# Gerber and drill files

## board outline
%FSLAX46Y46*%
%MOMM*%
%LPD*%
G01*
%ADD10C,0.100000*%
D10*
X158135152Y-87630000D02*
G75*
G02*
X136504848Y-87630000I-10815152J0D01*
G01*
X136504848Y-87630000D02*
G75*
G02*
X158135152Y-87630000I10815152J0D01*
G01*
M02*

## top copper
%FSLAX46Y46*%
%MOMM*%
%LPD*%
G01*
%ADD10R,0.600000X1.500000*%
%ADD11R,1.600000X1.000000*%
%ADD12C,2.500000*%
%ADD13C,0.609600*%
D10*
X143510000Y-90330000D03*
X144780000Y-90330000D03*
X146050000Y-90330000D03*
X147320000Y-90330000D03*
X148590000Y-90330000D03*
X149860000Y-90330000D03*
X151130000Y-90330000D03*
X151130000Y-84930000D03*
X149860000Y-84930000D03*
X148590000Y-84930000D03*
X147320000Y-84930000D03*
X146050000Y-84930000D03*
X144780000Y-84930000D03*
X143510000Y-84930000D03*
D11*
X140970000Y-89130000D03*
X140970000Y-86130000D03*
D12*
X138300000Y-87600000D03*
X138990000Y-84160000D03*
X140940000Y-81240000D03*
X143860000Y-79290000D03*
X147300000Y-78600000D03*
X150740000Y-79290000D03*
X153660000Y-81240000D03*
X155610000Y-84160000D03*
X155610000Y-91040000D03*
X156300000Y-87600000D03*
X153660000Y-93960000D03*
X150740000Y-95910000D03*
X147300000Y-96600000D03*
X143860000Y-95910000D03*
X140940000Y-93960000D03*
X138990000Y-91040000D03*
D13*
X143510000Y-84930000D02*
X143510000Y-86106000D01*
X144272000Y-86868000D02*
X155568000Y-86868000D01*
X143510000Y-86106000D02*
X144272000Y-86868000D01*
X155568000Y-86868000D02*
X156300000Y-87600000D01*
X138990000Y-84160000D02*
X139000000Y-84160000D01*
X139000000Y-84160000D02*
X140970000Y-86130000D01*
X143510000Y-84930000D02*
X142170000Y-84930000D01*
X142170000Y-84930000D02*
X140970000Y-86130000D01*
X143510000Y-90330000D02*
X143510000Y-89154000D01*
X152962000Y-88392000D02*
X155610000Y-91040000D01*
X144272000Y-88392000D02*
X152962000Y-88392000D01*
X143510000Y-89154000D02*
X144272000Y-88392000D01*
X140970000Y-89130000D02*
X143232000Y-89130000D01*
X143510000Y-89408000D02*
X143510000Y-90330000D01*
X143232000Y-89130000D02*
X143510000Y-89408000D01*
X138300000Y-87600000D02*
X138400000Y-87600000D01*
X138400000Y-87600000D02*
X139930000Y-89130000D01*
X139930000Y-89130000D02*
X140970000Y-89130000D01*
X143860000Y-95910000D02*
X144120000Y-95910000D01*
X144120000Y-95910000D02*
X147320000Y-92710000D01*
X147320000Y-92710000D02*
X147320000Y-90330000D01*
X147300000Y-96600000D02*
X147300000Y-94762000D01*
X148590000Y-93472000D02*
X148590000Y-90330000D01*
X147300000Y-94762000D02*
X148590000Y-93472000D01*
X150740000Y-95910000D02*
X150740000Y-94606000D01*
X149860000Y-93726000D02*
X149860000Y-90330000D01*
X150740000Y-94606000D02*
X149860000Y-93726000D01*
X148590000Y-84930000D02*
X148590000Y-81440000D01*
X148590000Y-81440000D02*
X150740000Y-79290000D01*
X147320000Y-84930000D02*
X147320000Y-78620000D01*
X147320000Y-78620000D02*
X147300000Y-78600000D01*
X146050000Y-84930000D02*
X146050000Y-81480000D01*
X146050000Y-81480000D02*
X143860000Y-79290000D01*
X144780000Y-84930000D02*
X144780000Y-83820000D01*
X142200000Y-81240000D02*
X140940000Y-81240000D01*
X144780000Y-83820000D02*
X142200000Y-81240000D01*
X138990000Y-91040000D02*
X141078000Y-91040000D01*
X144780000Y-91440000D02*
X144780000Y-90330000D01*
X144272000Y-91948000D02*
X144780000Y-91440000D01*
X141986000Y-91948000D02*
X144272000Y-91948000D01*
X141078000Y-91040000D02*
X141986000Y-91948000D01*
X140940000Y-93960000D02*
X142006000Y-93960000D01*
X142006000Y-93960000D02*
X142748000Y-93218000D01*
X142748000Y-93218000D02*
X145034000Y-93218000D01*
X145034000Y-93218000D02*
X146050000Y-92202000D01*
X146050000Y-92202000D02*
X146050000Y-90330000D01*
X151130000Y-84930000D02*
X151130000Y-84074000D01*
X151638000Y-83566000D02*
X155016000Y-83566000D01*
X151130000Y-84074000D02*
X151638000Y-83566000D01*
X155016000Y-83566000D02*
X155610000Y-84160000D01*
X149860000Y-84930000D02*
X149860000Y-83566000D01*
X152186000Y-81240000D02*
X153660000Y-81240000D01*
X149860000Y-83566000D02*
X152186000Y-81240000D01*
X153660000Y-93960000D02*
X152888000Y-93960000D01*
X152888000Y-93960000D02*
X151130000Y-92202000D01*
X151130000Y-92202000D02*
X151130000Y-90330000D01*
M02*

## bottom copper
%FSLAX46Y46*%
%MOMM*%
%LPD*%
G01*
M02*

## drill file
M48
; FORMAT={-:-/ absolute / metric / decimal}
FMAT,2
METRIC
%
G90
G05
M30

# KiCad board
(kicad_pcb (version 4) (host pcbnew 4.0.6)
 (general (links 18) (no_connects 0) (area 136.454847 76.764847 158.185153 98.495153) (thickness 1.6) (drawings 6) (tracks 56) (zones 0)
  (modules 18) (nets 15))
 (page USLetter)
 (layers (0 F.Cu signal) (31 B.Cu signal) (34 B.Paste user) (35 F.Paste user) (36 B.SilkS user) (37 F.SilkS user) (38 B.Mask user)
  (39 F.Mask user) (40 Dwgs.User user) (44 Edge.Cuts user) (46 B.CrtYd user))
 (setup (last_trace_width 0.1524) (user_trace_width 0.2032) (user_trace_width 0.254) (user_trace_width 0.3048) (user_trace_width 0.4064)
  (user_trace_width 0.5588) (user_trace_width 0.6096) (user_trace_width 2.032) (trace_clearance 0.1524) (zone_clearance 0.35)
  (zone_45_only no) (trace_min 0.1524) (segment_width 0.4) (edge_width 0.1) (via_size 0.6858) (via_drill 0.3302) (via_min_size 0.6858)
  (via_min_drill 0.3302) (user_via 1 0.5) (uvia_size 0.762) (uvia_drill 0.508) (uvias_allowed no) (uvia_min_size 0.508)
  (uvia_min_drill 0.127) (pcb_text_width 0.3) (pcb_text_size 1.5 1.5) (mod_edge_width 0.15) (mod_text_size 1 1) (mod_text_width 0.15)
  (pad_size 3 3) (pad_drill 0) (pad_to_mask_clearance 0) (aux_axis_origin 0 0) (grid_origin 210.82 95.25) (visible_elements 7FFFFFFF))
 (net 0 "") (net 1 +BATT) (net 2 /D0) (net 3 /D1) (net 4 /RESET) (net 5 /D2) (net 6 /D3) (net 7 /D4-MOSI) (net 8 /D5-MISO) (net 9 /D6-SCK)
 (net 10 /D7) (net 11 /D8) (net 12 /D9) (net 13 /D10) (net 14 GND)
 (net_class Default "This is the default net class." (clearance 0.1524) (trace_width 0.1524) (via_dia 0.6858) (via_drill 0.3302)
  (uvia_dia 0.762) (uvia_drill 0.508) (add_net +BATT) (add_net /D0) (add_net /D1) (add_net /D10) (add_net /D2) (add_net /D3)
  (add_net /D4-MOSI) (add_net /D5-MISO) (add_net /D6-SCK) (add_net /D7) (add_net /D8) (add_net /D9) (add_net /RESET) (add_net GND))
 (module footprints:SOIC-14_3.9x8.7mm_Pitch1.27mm (layer F.Cu) (at 147.32 87.63 90)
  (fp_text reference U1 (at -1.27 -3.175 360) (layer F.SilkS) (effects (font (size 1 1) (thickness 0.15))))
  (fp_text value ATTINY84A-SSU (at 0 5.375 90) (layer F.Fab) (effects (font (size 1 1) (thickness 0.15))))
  (pad 1 smd rect (at -2.7 -3.81 90) (size 1.5 0.6) (layers F.Cu F.Paste F.Mask) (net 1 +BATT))
  (pad 2 smd rect (at -2.7 -2.54 90) (size 1.5 0.6) (layers F.Cu F.Paste F.Mask) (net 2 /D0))
  (pad 3 smd rect (at -2.7 -1.27 90) (size 1.5 0.6) (layers F.Cu F.Paste F.Mask) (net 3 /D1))
  (pad 4 smd rect (at -2.7 0 90) (size 1.5 0.6) (layers F.Cu F.Paste F.Mask) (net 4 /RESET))
  (pad 5 smd rect (at -2.7 1.27 90) (size 1.5 0.6) (layers F.Cu F.Paste F.Mask) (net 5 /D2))
  (pad 6 smd rect (at -2.7 2.54 90) (size 1.5 0.6) (layers F.Cu F.Paste F.Mask) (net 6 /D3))
  (pad 7 smd rect (at -2.7 3.81 90) (size 1.5 0.6) (layers F.Cu F.Paste F.Mask) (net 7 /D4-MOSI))
  (pad 8 smd rect (at 2.7 3.81 90) (size 1.5 0.6) (layers F.Cu F.Paste F.Mask) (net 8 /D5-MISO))
  (pad 9 smd rect (at 2.7 2.54 90) (size 1.5 0.6) (layers F.Cu F.Paste F.Mask) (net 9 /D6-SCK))
  (pad 10 smd rect (at 2.7 1.27 90) (size 1.5 0.6) (layers F.Cu F.Paste F.Mask) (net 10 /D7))
  (pad 11 smd rect (at 2.7 0 90) (size 1.5 0.6) (layers F.Cu F.Paste F.Mask) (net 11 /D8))
  (pad 12 smd rect (at 2.7 -1.27 90) (size 1.5 0.6) (layers F.Cu F.Paste F.Mask) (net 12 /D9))
  (pad 13 smd rect (at 2.7 -2.54 90) (size 1.5 0.6) (layers F.Cu F.Paste F.Mask) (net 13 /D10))
  (pad 14 smd rect (at 2.7 -3.81 90) (size 1.5 0.6) (layers F.Cu F.Paste F.Mask) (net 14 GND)))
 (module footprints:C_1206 (layer F.Cu) (at 140.97 87.63 90)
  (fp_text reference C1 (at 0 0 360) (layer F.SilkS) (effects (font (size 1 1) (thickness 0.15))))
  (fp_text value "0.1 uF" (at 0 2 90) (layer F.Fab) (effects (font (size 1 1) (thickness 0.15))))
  (pad 1 smd rect (at -1.5 0 90) (size 1 1.6) (layers F.Cu F.Paste F.Mask) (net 1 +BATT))
  (pad 2 smd rect (at 1.5 0 90) (size 1 1.6) (layers F.Cu F.Paste F.Mask) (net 14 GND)))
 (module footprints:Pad (layer F.Cu) (at 138.3 87.6)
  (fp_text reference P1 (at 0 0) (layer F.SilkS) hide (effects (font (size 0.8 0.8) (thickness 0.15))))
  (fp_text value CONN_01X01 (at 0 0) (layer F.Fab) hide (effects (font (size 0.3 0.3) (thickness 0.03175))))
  (pad 1 smd circle (at 0 0) (size 2.5 2.5) (layers F.Cu F.Paste F.Mask) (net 1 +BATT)))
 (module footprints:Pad (layer F.Cu) (at 138.99 84.16)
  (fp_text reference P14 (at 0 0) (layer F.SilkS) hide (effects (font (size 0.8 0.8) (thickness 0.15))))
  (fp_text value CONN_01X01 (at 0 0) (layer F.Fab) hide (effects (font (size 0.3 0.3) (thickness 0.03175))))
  (pad 1 smd circle (at 0 0) (size 2.5 2.5) (layers F.Cu F.Paste F.Mask) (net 14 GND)))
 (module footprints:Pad (layer F.Cu) (at 140.94 81.24)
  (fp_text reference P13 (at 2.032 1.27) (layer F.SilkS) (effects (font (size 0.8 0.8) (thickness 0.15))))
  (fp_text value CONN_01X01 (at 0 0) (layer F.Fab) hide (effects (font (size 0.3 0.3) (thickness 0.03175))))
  (pad 1 smd circle (at 0 0) (size 2.5 2.5) (layers F.Cu F.Paste F.Mask) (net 13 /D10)))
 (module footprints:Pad (layer F.Cu) (at 143.86 79.29)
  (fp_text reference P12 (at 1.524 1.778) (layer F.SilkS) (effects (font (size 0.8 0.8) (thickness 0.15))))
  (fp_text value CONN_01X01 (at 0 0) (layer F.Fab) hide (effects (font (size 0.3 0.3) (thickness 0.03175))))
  (pad 1 smd circle (at 0 0) (size 2.5 2.5) (layers F.Cu F.Paste F.Mask) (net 12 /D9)))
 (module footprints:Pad (layer F.Cu) (at 147.3 78.6)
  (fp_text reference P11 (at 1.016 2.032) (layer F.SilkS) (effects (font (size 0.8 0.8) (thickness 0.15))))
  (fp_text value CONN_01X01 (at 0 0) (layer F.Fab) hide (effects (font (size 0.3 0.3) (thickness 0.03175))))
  (pad 1 smd circle (at 0 0) (size 2.5 2.5) (layers F.Cu F.Paste F.Mask) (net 11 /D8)))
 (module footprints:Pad (layer F.Cu) (at 150.74 79.29)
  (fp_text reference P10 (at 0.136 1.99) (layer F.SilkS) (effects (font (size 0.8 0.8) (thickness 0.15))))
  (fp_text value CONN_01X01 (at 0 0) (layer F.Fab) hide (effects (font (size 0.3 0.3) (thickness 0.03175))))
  (pad 1 smd circle (at 0 0) (size 2.5 2.5) (layers F.Cu F.Paste F.Mask) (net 10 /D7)))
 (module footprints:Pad (layer F.Cu) (at 153.66 81.24)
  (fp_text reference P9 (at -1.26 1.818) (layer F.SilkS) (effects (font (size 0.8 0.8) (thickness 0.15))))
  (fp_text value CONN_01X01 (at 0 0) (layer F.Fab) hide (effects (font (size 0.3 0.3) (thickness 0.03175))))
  (pad 1 smd circle (at 0 0) (size 2.5 2.5) (layers F.Cu F.Paste F.Mask) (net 9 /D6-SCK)))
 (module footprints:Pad (layer F.Cu) (at 155.61 84.16)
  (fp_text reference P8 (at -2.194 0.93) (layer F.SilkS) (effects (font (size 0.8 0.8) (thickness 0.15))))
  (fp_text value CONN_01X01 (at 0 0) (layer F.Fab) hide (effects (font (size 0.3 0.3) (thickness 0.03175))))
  (pad 1 smd circle (at 0 0) (size 2.5 2.5) (layers F.Cu F.Paste F.Mask) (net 8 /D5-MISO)))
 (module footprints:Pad (layer F.Cu) (at 155.61 91.04)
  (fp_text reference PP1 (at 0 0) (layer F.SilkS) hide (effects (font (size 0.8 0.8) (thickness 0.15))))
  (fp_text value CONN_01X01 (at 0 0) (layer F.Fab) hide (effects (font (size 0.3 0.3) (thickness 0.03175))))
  (pad 1 smd circle (at 0 0) (size 2.5 2.5) (layers F.Cu F.Paste F.Mask) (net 1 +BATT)))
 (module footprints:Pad (layer F.Cu) (at 156.3 87.6)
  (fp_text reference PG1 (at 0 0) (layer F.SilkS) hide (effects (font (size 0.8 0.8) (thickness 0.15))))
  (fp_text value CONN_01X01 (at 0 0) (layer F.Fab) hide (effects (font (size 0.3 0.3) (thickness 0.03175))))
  (pad 1 smd circle (at 0 0) (size 2.5 2.5) (layers F.Cu F.Paste F.Mask) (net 14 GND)))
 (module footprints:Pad (layer F.Cu) (at 153.66 93.96)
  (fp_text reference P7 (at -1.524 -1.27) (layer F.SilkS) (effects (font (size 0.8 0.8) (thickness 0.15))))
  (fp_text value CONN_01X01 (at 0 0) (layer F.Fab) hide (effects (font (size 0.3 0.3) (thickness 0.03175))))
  (pad 1 smd circle (at 0 0) (size 2.5 2.5) (layers F.Cu F.Paste F.Mask) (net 7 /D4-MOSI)))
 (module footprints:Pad (layer F.Cu) (at 150.74 95.91)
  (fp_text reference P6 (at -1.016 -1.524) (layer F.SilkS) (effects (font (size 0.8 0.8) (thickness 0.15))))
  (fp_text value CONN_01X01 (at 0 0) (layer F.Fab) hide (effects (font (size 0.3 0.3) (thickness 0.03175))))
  (pad 1 smd circle (at 0 0) (size 2.5 2.5) (layers F.Cu F.Paste F.Mask) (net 6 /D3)))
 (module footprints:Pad (layer F.Cu) (at 147.3 96.6)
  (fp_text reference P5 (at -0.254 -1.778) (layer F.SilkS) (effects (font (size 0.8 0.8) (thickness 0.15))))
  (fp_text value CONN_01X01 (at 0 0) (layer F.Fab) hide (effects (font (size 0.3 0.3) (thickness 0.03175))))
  (pad 1 smd circle (at 0 0) (size 2.5 2.5) (layers F.Cu F.Paste F.Mask) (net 5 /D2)))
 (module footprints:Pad (layer F.Cu) (at 143.86 95.91)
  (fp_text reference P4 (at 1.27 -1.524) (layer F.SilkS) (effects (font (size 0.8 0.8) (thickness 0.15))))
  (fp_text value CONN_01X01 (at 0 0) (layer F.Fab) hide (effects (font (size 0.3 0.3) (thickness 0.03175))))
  (pad 1 smd circle (at 0 0) (size 2.5 2.5) (layers F.Cu F.Paste F.Mask) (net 4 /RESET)))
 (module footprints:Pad (layer F.Cu) (at 140.94 93.96)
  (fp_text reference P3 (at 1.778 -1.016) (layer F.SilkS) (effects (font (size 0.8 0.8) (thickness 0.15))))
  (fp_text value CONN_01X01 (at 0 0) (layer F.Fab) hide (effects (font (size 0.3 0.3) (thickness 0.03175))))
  (pad 1 smd circle (at 0 0) (size 2.5 2.5) (layers F.Cu F.Paste F.Mask) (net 3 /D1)))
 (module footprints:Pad (layer F.Cu) (at 138.99 91.04)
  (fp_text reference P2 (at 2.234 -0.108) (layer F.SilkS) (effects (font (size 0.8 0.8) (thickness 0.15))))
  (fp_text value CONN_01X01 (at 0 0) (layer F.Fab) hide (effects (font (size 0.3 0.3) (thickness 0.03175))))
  (pad 1 smd circle (at 0 0) (size 2.5 2.5) (layers F.Cu F.Paste F.Mask) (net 2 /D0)))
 (gr_circle (center 147.32 87.63) (end 149.098 98.298) (layer Edge.Cuts) (width 0.1))
 (segment (start 143.51 84.93) (end 143.51 86.106) (width 0.6096) (layer F.Cu) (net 14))
 (segment (start 144.272 86.868) (end 155.568 86.868) (width 0.6096) (layer F.Cu) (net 14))
 (segment (start 143.51 86.106) (end 144.272 86.868) (width 0.6096) (layer F.Cu) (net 14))
 (segment (start 155.568 86.868) (end 156.3 87.6) (width 0.6096) (layer F.Cu) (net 14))
 (segment (start 138.99 84.16) (end 139 84.16) (width 0.6096) (layer F.Cu) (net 14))
 (segment (start 139 84.16) (end 140.97 86.13) (width 0.6096) (layer F.Cu) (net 14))
 (segment (start 143.51 84.93) (end 142.17 84.93) (width 0.6096) (layer F.Cu) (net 14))
 (segment (start 142.17 84.93) (end 140.97 86.13) (width 0.6096) (layer F.Cu) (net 14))
 (segment (start 143.51 90.33) (end 143.51 89.154) (width 0.6096) (layer F.Cu) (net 1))
 (segment (start 152.962 88.392) (end 155.61 91.04) (width 0.6096) (layer F.Cu) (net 1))
 (segment (start 144.272 88.392) (end 152.962 88.392) (width 0.6096) (layer F.Cu) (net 1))
 (segment (start 143.51 89.154) (end 144.272 88.392) (width 0.6096) (layer F.Cu) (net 1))
 (segment (start 140.97 89.13) (end 143.232 89.13) (width 0.6096) (layer F.Cu) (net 1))
 (segment (start 143.51 89.408) (end 143.51 90.33) (width 0.6096) (layer F.Cu) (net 1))
 (segment (start 143.232 89.13) (end 143.51 89.408) (width 0.6096) (layer F.Cu) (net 1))
 (segment (start 138.3 87.6) (end 138.4 87.6) (width 0.6096) (layer F.Cu) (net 1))
 (segment (start 138.4 87.6) (end 139.93 89.13) (width 0.6096) (layer F.Cu) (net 1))
 (segment (start 139.93 89.13) (end 140.97 89.13) (width 0.6096) (layer F.Cu) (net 1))
 (segment (start 143.86 95.91) (end 144.12 95.91) (width 0.6096) (layer F.Cu) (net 4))
 (segment (start 144.12 95.91) (end 147.32 92.71) (width 0.6096) (layer F.Cu) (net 4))
 (segment (start 147.32 92.71) (end 147.32 90.33) (width 0.6096) (layer F.Cu) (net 4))
 (segment (start 147.3 96.6) (end 147.3 94.762) (width 0.6096) (layer F.Cu) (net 5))
 (segment (start 148.59 93.472) (end 148.59 90.33) (width 0.6096) (layer F.Cu) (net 5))
 (segment (start 147.3 94.762) (end 148.59 93.472) (width 0.6096) (layer F.Cu) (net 5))
 (segment (start 150.74 95.91) (end 150.74 94.606) (width 0.6096) (layer F.Cu) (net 6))
 (segment (start 149.86 93.726) (end 149.86 90.33) (width 0.6096) (layer F.Cu) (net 6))
 (segment (start 150.74 94.606) (end 149.86 93.726) (width 0.6096) (layer F.Cu) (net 6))
 (segment (start 148.59 84.93) (end 148.59 81.44) (width 0.6096) (layer F.Cu) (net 10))
 (segment (start 148.59 81.44) (end 150.74 79.29) (width 0.6096) (layer F.Cu) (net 10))
 (segment (start 147.32 84.93) (end 147.32 78.62) (width 0.6096) (layer F.Cu) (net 11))
 (segment (start 147.32 78.62) (end 147.3 78.6) (width 0.6096) (layer F.Cu) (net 11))
 (segment (start 146.05 84.93) (end 146.05 81.48) (width 0.6096) (layer F.Cu) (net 12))
 (segment (start 146.05 81.48) (end 143.86 79.29) (width 0.6096) (layer F.Cu) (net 12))
 (segment (start 144.78 84.93) (end 144.78 83.82) (width 0.6096) (layer F.Cu) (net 13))
 (segment (start 142.2 81.24) (end 140.94 81.24) (width 0.6096) (layer F.Cu) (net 13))
 (segment (start 144.78 83.82) (end 142.2 81.24) (width 0.6096) (layer F.Cu) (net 13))
 (segment (start 138.99 91.04) (end 141.078 91.04) (width 0.6096) (layer F.Cu) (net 2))
 (segment (start 144.78 91.44) (end 144.78 90.33) (width 0.6096) (layer F.Cu) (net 2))
 (segment (start 144.272 91.948) (end 144.78 91.44) (width 0.6096) (layer F.Cu) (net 2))
 (segment (start 141.986 91.948) (end 144.272 91.948) (width 0.6096) (layer F.Cu) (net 2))
 (segment (start 141.078 91.04) (end 141.986 91.948) (width 0.6096) (layer F.Cu) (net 2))
 (segment (start 140.94 93.96) (end 142.006 93.96) (width 0.6096) (layer F.Cu) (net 3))
 (segment (start 142.006 93.96) (end 142.748 93.218) (width 0.6096) (layer F.Cu) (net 3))
 (segment (start 142.748 93.218) (end 145.034 93.218) (width 0.6096) (layer F.Cu) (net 3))
 (segment (start 145.034 93.218) (end 146.05 92.202) (width 0.6096) (layer F.Cu) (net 3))
 (segment (start 146.05 92.202) (end 146.05 90.33) (width 0.6096) (layer F.Cu) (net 3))
 (segment (start 151.13 84.93) (end 151.13 84.074) (width 0.6096) (layer F.Cu) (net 8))
 (segment (start 151.638 83.566) (end 155.016 83.566) (width 0.6096) (layer F.Cu) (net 8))
 (segment (start 151.13 84.074) (end 151.638 83.566) (width 0.6096) (layer F.Cu) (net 8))
 (segment (start 155.016 83.566) (end 155.61 84.16) (width 0.6096) (layer F.Cu) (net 8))
 (segment (start 149.86 84.93) (end 149.86 83.566) (width 0.6096) (layer F.Cu) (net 9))
 (segment (start 152.186 81.24) (end 153.66 81.24) (width 0.6096) (layer F.Cu) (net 9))
 (segment (start 149.86 83.566) (end 152.186 81.24) (width 0.6096) (layer F.Cu) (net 9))
 (segment (start 153.66 93.96) (end 152.888 93.96) (width 0.6096) (layer F.Cu) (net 7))
 (segment (start 152.888 93.96) (end 151.13 92.202) (width 0.6096) (layer F.Cu) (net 7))
 (segment (start 151.13 92.202) (end 151.13 90.33) (width 0.6096) (layer F.Cu) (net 7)))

